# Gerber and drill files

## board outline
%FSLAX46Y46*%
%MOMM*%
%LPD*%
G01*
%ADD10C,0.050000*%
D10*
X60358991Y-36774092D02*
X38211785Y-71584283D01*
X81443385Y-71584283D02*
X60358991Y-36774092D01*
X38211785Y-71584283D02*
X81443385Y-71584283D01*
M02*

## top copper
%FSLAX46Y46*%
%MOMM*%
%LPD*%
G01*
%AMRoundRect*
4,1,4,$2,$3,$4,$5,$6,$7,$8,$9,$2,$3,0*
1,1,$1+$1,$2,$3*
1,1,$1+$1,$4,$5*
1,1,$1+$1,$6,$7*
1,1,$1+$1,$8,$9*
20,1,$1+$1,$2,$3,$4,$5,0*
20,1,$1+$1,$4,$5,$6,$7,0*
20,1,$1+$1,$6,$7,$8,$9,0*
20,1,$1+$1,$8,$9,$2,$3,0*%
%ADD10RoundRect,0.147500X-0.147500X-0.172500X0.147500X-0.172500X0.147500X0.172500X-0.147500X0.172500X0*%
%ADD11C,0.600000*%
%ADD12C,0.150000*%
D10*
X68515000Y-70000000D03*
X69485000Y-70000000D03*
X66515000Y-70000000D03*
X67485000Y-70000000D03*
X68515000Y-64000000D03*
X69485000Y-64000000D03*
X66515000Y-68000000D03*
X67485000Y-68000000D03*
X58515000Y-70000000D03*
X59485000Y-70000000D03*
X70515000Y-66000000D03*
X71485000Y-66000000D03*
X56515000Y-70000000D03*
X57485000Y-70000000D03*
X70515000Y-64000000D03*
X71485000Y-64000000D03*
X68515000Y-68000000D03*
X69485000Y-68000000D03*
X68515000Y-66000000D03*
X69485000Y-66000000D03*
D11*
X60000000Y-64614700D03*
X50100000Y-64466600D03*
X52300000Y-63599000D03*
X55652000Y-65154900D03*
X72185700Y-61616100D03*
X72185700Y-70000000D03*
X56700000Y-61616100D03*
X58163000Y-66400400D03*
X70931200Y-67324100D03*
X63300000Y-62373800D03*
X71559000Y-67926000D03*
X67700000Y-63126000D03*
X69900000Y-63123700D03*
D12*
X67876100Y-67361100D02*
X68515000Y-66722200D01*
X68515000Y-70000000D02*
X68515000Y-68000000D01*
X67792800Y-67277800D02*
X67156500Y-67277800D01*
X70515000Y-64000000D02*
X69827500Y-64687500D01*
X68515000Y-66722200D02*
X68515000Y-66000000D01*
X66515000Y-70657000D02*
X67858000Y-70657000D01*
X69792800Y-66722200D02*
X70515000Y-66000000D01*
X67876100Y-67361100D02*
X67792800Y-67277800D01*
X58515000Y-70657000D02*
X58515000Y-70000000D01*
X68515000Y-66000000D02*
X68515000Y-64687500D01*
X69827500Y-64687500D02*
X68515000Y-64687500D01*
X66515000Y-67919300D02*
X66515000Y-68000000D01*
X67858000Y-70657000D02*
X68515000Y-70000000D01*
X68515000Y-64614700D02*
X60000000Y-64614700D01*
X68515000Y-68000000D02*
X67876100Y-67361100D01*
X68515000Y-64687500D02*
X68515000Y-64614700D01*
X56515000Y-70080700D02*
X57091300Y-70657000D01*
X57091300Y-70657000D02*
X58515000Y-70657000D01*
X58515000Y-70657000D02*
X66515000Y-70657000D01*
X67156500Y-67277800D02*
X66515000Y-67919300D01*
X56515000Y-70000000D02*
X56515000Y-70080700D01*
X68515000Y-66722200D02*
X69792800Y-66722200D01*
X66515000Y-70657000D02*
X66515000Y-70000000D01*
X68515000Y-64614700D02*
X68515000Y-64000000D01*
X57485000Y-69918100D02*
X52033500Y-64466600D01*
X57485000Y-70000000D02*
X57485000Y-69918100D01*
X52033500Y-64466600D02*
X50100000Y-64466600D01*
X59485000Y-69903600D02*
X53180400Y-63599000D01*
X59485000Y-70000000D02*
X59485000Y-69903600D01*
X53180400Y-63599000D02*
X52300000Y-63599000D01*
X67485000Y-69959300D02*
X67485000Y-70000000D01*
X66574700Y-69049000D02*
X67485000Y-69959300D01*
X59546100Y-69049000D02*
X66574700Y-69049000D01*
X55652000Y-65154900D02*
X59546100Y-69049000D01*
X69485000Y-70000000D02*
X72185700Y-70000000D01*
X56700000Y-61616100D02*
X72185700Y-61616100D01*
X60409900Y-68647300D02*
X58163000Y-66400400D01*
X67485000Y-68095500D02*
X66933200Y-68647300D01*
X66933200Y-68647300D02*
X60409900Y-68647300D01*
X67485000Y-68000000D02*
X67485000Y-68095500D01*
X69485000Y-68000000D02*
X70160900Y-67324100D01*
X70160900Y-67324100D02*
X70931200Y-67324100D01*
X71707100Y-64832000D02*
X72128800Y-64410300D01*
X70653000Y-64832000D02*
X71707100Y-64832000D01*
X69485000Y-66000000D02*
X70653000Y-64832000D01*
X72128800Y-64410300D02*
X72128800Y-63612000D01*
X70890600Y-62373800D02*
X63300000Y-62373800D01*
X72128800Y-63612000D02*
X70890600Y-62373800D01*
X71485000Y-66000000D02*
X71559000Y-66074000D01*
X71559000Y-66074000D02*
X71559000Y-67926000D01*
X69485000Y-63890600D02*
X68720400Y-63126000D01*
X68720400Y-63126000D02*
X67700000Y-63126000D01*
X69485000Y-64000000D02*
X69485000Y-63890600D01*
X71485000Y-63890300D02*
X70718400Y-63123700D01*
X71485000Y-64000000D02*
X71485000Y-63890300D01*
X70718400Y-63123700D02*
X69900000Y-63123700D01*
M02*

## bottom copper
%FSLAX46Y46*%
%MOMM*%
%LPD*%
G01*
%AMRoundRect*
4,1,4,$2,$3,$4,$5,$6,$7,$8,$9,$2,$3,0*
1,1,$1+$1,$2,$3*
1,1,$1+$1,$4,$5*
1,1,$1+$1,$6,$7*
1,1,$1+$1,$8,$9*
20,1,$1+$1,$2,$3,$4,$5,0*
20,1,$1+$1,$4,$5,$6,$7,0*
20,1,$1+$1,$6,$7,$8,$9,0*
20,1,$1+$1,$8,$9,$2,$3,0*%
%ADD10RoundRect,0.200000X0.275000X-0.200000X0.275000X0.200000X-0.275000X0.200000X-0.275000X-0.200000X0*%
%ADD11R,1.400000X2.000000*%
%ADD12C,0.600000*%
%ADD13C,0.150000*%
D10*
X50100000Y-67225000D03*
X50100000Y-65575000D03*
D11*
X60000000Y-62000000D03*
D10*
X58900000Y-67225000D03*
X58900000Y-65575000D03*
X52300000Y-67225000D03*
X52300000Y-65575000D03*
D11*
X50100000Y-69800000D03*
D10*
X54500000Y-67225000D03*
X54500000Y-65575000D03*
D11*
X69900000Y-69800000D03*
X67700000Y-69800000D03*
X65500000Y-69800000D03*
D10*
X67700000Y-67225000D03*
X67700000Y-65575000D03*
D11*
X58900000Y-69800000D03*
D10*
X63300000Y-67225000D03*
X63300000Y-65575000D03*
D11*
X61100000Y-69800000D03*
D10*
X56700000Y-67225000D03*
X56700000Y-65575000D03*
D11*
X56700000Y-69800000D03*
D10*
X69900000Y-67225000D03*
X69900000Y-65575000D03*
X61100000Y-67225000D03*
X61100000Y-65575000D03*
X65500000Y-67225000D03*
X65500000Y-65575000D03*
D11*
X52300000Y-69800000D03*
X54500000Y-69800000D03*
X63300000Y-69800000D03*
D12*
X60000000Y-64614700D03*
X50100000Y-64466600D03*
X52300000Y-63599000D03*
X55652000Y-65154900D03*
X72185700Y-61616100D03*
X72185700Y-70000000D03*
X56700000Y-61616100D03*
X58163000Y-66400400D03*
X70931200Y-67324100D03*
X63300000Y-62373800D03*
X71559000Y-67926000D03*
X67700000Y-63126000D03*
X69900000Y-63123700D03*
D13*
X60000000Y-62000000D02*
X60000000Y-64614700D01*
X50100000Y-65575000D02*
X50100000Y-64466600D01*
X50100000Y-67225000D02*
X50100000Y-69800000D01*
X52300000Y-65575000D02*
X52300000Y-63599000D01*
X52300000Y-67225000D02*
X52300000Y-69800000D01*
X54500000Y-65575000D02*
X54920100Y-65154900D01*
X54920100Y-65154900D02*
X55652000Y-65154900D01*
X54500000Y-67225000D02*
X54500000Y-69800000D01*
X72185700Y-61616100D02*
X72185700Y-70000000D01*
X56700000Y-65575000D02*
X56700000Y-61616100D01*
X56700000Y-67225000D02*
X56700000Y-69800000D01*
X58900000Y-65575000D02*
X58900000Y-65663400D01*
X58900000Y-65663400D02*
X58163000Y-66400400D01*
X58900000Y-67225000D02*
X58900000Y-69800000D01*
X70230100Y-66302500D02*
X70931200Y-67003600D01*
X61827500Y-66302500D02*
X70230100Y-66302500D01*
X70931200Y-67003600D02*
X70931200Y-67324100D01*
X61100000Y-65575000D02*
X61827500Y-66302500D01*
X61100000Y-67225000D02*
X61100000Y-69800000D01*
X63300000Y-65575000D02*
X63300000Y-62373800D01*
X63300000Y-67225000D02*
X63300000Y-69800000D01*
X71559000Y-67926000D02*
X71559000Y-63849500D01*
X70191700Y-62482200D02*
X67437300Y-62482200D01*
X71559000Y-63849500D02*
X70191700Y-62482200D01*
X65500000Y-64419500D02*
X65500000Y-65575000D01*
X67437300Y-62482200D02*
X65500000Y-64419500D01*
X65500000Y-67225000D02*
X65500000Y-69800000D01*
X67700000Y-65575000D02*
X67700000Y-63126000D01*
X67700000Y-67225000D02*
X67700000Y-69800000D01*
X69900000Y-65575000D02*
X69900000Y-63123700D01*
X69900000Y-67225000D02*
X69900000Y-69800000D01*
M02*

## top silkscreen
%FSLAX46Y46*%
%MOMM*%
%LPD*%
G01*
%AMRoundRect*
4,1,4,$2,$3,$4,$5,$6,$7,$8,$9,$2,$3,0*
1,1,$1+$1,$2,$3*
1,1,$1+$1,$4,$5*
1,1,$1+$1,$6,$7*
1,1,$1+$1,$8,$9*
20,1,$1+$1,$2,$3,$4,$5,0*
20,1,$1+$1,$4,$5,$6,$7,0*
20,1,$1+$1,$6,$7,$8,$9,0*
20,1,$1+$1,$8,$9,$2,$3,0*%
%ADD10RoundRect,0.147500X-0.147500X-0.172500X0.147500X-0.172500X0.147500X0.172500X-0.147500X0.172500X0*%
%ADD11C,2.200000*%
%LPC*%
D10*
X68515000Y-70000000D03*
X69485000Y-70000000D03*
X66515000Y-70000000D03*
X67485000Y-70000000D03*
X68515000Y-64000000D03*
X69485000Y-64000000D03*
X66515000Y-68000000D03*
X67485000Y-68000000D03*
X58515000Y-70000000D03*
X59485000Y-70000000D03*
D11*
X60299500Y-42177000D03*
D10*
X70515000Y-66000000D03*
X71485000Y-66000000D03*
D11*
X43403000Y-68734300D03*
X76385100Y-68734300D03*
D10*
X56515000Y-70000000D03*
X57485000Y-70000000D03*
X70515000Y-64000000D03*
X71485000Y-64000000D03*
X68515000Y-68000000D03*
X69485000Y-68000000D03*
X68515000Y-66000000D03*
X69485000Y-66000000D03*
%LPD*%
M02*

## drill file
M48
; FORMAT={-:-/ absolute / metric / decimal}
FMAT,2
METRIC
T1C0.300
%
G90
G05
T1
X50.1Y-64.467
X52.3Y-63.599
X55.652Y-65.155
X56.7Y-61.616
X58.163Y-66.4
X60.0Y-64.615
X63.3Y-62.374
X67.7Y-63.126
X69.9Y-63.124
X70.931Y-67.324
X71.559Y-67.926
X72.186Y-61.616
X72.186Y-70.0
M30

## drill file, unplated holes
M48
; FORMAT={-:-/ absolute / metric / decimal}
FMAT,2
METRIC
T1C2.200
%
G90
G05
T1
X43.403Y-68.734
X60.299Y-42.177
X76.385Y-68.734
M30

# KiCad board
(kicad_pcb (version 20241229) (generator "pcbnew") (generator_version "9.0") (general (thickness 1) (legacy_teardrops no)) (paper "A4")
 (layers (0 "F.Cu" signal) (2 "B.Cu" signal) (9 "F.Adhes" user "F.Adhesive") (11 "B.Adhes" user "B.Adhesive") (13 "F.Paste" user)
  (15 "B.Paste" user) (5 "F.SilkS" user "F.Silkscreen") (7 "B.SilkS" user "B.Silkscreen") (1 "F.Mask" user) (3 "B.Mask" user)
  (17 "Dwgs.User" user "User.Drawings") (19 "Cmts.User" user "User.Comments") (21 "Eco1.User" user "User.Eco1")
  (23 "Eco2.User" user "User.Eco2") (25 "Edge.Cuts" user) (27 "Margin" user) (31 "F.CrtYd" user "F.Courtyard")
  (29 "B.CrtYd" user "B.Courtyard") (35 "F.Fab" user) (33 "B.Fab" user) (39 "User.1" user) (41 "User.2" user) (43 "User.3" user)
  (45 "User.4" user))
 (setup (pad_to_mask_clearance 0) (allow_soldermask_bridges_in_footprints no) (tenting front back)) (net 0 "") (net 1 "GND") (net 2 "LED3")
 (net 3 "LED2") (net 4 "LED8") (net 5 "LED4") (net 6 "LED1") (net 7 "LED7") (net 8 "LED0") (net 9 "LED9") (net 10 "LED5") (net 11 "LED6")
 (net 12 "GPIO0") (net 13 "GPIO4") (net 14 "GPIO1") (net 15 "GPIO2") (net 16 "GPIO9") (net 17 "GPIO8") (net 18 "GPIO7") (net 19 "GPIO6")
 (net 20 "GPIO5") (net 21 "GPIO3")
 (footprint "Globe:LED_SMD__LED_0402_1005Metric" (layer "F.Cu") (at 69 70)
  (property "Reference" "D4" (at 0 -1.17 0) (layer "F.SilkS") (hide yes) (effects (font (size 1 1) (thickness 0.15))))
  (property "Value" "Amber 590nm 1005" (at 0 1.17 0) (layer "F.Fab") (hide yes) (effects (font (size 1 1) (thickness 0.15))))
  (pad "1" smd roundrect (at -0.485 0) (size 0.59 0.64) (layers "F.Cu" "F.Mask" "F.Paste") (roundrect_rratio 0.25) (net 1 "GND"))
  (pad "2" smd roundrect (at 0.485 0) (size 0.59 0.64) (layers "F.Cu" "F.Mask" "F.Paste") (roundrect_rratio 0.25) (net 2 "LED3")))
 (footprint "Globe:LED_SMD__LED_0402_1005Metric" (layer "F.Cu") (at 67 70)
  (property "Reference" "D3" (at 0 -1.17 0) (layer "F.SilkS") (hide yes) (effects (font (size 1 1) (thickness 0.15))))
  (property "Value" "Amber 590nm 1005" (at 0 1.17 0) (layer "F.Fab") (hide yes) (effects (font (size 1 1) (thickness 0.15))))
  (pad "1" smd roundrect (at -0.485 0) (size 0.59 0.64) (layers "F.Cu" "F.Mask" "F.Paste") (roundrect_rratio 0.25) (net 1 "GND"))
  (pad "2" smd roundrect (at 0.485 0) (size 0.59 0.64) (layers "F.Cu" "F.Mask" "F.Paste") (roundrect_rratio 0.25) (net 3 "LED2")))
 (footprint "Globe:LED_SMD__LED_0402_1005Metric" (layer "F.Cu") (at 69 64)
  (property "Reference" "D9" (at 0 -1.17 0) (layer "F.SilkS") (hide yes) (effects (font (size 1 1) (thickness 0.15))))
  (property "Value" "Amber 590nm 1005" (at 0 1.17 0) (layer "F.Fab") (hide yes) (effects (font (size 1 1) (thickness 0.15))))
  (pad "1" smd roundrect (at -0.485 0) (size 0.59 0.64) (layers "F.Cu" "F.Mask" "F.Paste") (roundrect_rratio 0.25) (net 1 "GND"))
  (pad "2" smd roundrect (at 0.485 0) (size 0.59 0.64) (layers "F.Cu" "F.Mask" "F.Paste") (roundrect_rratio 0.25) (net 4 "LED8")))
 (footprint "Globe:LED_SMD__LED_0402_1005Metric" (layer "F.Cu") (at 67 68)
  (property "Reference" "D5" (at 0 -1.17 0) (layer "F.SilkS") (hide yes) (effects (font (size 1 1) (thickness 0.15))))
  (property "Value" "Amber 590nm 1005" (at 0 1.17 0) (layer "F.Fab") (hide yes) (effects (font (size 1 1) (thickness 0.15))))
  (pad "1" smd roundrect (at -0.485 0) (size 0.59 0.64) (layers "F.Cu" "F.Mask" "F.Paste") (roundrect_rratio 0.25) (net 1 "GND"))
  (pad "2" smd roundrect (at 0.485 0) (size 0.59 0.64) (layers "F.Cu" "F.Mask" "F.Paste") (roundrect_rratio 0.25) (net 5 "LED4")))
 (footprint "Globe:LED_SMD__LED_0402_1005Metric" (layer "F.Cu") (at 59 70)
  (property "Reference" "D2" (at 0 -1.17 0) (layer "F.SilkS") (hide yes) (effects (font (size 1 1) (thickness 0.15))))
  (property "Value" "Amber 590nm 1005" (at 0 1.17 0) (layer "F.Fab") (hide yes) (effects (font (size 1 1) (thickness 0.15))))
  (pad "1" smd roundrect (at -0.485 0) (size 0.59 0.64) (layers "F.Cu" "F.Mask" "F.Paste") (roundrect_rratio 0.25) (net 1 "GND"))
  (pad "2" smd roundrect (at 0.485 0) (size 0.59 0.64) (layers "F.Cu" "F.Mask" "F.Paste") (roundrect_rratio 0.25) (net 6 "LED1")))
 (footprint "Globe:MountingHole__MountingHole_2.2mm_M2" (layer "F.Cu") (at 60.2995 42.177)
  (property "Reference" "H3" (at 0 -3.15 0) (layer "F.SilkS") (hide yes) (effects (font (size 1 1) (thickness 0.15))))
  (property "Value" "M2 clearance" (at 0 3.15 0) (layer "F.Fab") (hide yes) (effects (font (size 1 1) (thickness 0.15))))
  (pad "" np_thru_hole circle (at 0 0) (size 2.2 2.2) (drill 2.2) (layers "*.Cu" "*.Mask")))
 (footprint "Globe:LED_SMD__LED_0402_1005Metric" (layer "F.Cu") (at 71 66)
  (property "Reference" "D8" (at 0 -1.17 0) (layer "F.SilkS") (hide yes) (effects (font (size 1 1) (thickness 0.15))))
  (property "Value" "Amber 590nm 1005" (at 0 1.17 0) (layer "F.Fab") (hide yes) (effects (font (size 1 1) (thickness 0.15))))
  (pad "1" smd roundrect (at -0.485 0) (size 0.59 0.64) (layers "F.Cu" "F.Mask" "F.Paste") (roundrect_rratio 0.25) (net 1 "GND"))
  (pad "2" smd roundrect (at 0.485 0) (size 0.59 0.64) (layers "F.Cu" "F.Mask" "F.Paste") (roundrect_rratio 0.25) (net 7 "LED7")))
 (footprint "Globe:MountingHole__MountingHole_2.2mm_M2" (layer "F.Cu") (at 43.403 68.7343)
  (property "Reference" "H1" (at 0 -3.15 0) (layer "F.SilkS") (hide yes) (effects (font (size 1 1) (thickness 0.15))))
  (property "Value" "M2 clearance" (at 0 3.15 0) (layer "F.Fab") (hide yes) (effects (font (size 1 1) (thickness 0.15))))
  (pad "" np_thru_hole circle (at 0 0) (size 2.2 2.2) (drill 2.2) (layers "*.Cu" "*.Mask")))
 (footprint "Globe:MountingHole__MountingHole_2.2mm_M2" (layer "F.Cu") (at 76.3851 68.7343)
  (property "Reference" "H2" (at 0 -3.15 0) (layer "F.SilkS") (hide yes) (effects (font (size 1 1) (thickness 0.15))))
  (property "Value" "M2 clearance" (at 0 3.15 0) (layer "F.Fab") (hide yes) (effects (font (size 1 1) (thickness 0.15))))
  (pad "" np_thru_hole circle (at 0 0) (size 2.2 2.2) (drill 2.2) (layers "*.Cu" "*.Mask")))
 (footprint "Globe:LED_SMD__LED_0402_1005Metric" (layer "F.Cu") (at 57 70)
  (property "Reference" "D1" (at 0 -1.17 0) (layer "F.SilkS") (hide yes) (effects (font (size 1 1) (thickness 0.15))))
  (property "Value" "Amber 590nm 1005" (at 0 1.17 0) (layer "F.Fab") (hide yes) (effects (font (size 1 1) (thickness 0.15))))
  (pad "1" smd roundrect (at -0.485 0) (size 0.59 0.64) (layers "F.Cu" "F.Mask" "F.Paste") (roundrect_rratio 0.25) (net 1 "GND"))
  (pad "2" smd roundrect (at 0.485 0) (size 0.59 0.64) (layers "F.Cu" "F.Mask" "F.Paste") (roundrect_rratio 0.25) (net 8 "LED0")))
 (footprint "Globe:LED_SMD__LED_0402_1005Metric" (layer "F.Cu") (at 71 64)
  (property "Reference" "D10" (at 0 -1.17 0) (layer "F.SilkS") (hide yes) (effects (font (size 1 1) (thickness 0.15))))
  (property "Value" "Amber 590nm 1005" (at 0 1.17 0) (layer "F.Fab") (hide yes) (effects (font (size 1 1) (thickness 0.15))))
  (pad "1" smd roundrect (at -0.485 0) (size 0.59 0.64) (layers "F.Cu" "F.Mask" "F.Paste") (roundrect_rratio 0.25) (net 1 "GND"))
  (pad "2" smd roundrect (at 0.485 0) (size 0.59 0.64) (layers "F.Cu" "F.Mask" "F.Paste") (roundrect_rratio 0.25) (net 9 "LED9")))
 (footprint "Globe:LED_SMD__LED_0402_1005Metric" (layer "F.Cu") (at 69 68)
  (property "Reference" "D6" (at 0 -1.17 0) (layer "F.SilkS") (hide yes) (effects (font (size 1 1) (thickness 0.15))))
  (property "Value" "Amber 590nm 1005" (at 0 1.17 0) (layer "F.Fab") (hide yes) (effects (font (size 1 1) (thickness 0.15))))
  (pad "1" smd roundrect (at -0.485 0) (size 0.59 0.64) (layers "F.Cu" "F.Mask" "F.Paste") (roundrect_rratio 0.25) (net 1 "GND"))
  (pad "2" smd roundrect (at 0.485 0) (size 0.59 0.64) (layers "F.Cu" "F.Mask" "F.Paste") (roundrect_rratio 0.25) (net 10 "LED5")))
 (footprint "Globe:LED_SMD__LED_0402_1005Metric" (layer "F.Cu") (at 69 66)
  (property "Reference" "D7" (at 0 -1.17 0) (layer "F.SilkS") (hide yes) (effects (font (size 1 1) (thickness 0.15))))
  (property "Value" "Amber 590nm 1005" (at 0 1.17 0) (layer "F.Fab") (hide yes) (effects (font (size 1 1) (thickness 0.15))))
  (pad "1" smd roundrect (at -0.485 0) (size 0.59 0.64) (layers "F.Cu" "F.Mask" "F.Paste") (roundrect_rratio 0.25) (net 1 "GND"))
  (pad "2" smd roundrect (at 0.485 0) (size 0.59 0.64) (layers "F.Cu" "F.Mask" "F.Paste") (roundrect_rratio 0.25) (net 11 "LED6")))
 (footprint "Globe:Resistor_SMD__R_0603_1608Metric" (layer "B.Cu") (at 50.1 66.4 90)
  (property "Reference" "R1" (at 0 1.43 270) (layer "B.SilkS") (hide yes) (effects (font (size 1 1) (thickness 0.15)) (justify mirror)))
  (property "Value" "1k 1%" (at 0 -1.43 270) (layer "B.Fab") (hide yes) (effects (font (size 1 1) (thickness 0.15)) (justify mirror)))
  (pad "1" smd roundrect (at -0.825 0 90) (size 0.8 0.95) (layers "B.Cu" "B.Mask" "B.Paste") (roundrect_rratio 0.25) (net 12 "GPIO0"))
  (pad "2" smd roundrect (at 0.825 0 90) (size 0.8 0.95) (layers "B.Cu" "B.Mask" "B.Paste") (roundrect_rratio 0.25) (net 8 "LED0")))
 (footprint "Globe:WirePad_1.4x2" (layer "B.Cu") (at 60 62 180)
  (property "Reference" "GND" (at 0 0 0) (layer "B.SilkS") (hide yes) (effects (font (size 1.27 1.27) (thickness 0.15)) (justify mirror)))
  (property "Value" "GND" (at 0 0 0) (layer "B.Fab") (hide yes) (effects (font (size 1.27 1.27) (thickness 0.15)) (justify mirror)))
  (pad "1" smd rect (at 0 0 180) (size 1.4 2) (layers "B.Cu" "B.Mask") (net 1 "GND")))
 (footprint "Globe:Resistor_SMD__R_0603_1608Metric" (layer "B.Cu") (at 58.9 66.4 90)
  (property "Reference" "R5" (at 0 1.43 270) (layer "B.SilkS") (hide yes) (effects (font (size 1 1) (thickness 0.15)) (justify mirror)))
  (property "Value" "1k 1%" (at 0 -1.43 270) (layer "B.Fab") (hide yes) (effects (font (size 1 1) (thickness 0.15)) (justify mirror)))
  (pad "1" smd roundrect (at -0.825 0 90) (size 0.8 0.95) (layers "B.Cu" "B.Mask" "B.Paste") (roundrect_rratio 0.25) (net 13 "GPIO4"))
  (pad "2" smd roundrect (at 0.825 0 90) (size 0.8 0.95) (layers "B.Cu" "B.Mask" "B.Paste") (roundrect_rratio 0.25) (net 5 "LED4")))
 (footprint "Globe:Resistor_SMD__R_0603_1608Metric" (layer "B.Cu") (at 52.3 66.4 90)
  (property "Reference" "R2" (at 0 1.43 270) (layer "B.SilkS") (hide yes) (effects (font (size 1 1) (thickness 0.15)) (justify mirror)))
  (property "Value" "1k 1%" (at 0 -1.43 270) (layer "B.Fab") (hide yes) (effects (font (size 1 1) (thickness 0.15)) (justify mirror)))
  (pad "1" smd roundrect (at -0.825 0 90) (size 0.8 0.95) (layers "B.Cu" "B.Mask" "B.Paste") (roundrect_rratio 0.25) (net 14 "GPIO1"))
  (pad "2" smd roundrect (at 0.825 0 90) (size 0.8 0.95) (layers "B.Cu" "B.Mask" "B.Paste") (roundrect_rratio 0.25) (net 6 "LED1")))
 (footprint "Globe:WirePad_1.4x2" (layer "B.Cu") (at 50.1 69.8 180)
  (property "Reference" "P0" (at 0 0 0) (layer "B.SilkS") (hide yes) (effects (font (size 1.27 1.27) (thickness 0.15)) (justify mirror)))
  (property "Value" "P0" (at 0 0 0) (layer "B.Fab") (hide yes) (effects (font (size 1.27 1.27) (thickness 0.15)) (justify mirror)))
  (pad "1" smd rect (at 0 0 180) (size 1.4 2) (layers "B.Cu" "B.Mask") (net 12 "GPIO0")))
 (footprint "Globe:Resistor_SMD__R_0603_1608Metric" (layer "B.Cu") (at 54.5 66.4 90)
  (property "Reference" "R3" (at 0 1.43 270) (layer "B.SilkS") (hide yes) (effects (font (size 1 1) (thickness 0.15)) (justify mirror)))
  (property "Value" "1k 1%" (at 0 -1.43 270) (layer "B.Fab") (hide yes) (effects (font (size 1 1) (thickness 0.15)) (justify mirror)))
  (pad "1" smd roundrect (at -0.825 0 90) (size 0.8 0.95) (layers "B.Cu" "B.Mask" "B.Paste") (roundrect_rratio 0.25) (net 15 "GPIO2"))
  (pad "2" smd roundrect (at 0.825 0 90) (size 0.8 0.95) (layers "B.Cu" "B.Mask" "B.Paste") (roundrect_rratio 0.25) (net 3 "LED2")))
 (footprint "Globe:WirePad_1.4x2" (layer "B.Cu") (at 69.9 69.8 180)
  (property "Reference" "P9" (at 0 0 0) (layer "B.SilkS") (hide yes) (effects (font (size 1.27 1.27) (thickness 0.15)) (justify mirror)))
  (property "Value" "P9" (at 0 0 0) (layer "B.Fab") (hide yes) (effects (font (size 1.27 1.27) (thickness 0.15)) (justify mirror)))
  (pad "1" smd rect (at 0 0 180) (size 1.4 2) (layers "B.Cu" "B.Mask") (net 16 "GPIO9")))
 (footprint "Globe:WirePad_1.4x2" (layer "B.Cu") (at 67.7 69.8 180)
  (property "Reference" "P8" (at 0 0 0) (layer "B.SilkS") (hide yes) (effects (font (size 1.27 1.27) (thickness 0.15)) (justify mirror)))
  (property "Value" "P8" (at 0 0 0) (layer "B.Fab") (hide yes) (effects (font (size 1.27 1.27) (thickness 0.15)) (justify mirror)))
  (pad "1" smd rect (at 0 0 180) (size 1.4 2) (layers "B.Cu" "B.Mask") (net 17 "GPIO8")))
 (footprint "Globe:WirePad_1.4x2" (layer "B.Cu") (at 65.5 69.8 180)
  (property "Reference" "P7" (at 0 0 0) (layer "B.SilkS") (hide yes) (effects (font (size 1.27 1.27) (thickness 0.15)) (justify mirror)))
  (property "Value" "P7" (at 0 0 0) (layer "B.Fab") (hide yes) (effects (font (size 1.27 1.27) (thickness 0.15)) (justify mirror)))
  (pad "1" smd rect (at 0 0 180) (size 1.4 2) (layers "B.Cu" "B.Mask") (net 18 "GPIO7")))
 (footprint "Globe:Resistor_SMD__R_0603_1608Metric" (layer "B.Cu") (at 67.7 66.4 90)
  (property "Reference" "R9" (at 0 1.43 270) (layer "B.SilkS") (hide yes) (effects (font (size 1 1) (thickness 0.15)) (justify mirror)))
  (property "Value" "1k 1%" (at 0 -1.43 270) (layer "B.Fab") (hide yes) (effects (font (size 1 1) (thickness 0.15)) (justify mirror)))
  (pad "1" smd roundrect (at -0.825 0 90) (size 0.8 0.95) (layers "B.Cu" "B.Mask" "B.Paste") (roundrect_rratio 0.25) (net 17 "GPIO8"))
  (pad "2" smd roundrect (at 0.825 0 90) (size 0.8 0.95) (layers "B.Cu" "B.Mask" "B.Paste") (roundrect_rratio 0.25) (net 4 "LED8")))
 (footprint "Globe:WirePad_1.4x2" (layer "B.Cu") (at 58.9 69.8 180)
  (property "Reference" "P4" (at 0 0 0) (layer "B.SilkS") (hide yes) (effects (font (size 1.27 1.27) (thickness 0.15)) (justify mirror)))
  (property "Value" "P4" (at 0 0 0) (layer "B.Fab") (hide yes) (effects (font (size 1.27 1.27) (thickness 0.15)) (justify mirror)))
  (pad "1" smd rect (at 0 0 180) (size 1.4 2) (layers "B.Cu" "B.Mask") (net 13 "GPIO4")))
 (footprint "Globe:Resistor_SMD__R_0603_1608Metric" (layer "B.Cu") (at 63.3 66.4 90)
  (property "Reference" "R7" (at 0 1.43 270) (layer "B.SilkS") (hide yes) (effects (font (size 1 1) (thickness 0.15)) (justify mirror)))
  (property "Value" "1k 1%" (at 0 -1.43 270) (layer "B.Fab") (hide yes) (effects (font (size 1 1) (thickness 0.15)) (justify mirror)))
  (pad "1" smd roundrect (at -0.825 0 90) (size 0.8 0.95) (layers "B.Cu" "B.Mask" "B.Paste") (roundrect_rratio 0.25) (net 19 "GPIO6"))
  (pad "2" smd roundrect (at 0.825 0 90) (size 0.8 0.95) (layers "B.Cu" "B.Mask" "B.Paste") (roundrect_rratio 0.25) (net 11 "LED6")))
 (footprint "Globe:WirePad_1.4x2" (layer "B.Cu") (at 61.1 69.8 180)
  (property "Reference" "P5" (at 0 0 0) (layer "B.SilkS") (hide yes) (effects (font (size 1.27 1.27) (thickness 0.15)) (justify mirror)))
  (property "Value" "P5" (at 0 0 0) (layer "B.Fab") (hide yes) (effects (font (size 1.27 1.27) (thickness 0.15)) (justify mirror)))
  (pad "1" smd rect (at 0 0 180) (size 1.4 2) (layers "B.Cu" "B.Mask") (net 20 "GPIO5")))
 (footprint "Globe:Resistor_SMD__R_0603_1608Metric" (layer "B.Cu") (at 56.7 66.4 90)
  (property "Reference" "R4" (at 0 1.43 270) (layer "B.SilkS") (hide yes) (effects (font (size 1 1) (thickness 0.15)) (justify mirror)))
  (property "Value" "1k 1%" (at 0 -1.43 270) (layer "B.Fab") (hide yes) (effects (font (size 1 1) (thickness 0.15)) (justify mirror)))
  (pad "1" smd roundrect (at -0.825 0 90) (size 0.8 0.95) (layers "B.Cu" "B.Mask" "B.Paste") (roundrect_rratio 0.25) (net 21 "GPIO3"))
  (pad "2" smd roundrect (at 0.825 0 90) (size 0.8 0.95) (layers "B.Cu" "B.Mask" "B.Paste") (roundrect_rratio 0.25) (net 2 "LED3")))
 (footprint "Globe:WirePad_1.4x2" (layer "B.Cu") (at 56.7 69.8 180)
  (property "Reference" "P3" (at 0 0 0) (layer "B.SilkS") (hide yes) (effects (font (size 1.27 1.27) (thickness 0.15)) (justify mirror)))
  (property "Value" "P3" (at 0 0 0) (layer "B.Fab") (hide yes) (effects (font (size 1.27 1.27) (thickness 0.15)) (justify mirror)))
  (pad "1" smd rect (at 0 0 180) (size 1.4 2) (layers "B.Cu" "B.Mask") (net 21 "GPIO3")))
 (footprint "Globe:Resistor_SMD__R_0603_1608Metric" (layer "B.Cu") (at 69.9 66.4 90)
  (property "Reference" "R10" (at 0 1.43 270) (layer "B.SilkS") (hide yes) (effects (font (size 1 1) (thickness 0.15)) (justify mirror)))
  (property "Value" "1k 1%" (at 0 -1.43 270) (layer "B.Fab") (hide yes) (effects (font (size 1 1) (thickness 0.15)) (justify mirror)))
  (pad "1" smd roundrect (at -0.825 0 90) (size 0.8 0.95) (layers "B.Cu" "B.Mask" "B.Paste") (roundrect_rratio 0.25) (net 16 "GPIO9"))
  (pad "2" smd roundrect (at 0.825 0 90) (size 0.8 0.95) (layers "B.Cu" "B.Mask" "B.Paste") (roundrect_rratio 0.25) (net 9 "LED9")))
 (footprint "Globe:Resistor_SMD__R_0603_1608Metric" (layer "B.Cu") (at 61.1 66.4 90)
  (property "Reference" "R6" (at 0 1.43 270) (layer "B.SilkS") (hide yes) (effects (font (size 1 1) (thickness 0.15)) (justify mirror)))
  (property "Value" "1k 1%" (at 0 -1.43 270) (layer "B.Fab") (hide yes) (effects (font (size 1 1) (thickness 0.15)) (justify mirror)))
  (pad "1" smd roundrect (at -0.825 0 90) (size 0.8 0.95) (layers "B.Cu" "B.Mask" "B.Paste") (roundrect_rratio 0.25) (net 20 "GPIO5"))
  (pad "2" smd roundrect (at 0.825 0 90) (size 0.8 0.95) (layers "B.Cu" "B.Mask" "B.Paste") (roundrect_rratio 0.25) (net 10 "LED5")))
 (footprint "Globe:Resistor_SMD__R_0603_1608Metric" (layer "B.Cu") (at 65.5 66.4 90)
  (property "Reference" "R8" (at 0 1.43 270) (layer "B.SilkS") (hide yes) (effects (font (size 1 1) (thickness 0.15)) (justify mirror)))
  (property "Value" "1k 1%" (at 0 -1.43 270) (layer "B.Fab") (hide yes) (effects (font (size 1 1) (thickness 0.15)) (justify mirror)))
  (pad "1" smd roundrect (at -0.825 0 90) (size 0.8 0.95) (layers "B.Cu" "B.Mask" "B.Paste") (roundrect_rratio 0.25) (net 18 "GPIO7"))
  (pad "2" smd roundrect (at 0.825 0 90) (size 0.8 0.95) (layers "B.Cu" "B.Mask" "B.Paste") (roundrect_rratio 0.25) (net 7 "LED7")))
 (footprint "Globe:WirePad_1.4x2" (layer "B.Cu") (at 52.3 69.8 180)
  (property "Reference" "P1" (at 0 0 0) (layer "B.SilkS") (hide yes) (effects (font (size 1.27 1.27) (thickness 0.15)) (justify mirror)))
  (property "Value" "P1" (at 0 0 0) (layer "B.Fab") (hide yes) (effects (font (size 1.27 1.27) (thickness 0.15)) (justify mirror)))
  (pad "1" smd rect (at 0 0 180) (size 1.4 2) (layers "B.Cu" "B.Mask") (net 14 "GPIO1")))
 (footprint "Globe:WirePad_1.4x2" (layer "B.Cu") (at 54.5 69.8 180)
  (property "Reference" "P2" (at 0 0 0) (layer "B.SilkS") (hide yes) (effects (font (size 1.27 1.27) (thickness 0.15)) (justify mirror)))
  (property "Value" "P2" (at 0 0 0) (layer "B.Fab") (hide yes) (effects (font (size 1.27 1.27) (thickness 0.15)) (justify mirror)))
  (pad "1" smd rect (at 0 0 180) (size 1.4 2) (layers "B.Cu" "B.Mask") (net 15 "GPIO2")))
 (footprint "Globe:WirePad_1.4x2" (layer "B.Cu") (at 63.3 69.8 180)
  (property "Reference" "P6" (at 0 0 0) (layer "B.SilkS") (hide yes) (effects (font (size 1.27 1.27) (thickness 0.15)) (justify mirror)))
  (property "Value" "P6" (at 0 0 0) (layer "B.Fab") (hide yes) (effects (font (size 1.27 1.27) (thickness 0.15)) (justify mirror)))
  (pad "1" smd rect (at 0 0 180) (size 1.4 2) (layers "B.Cu" "B.Mask") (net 19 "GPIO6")))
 (gr_line (start 60.358991 36.774092) (end 38.211785 71.584283) (stroke (width 0.05) (type default)) (layer "Edge.Cuts"))
 (gr_line (start 81.443385 71.584283) (end 60.358991 36.774092) (stroke (width 0.05) (type default)) (layer "Edge.Cuts"))
 (gr_line (start 38.211785 71.584283) (end 81.443385 71.584283) (stroke (width 0.05) (type default)) (layer "Edge.Cuts"))
 (segment (start 67.8761 67.3611) (end 68.515 66.7222) (width 0.15) (layer "F.Cu") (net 1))
 (segment (start 68.515 70) (end 68.515 68) (width 0.15) (layer "F.Cu") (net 1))
 (segment (start 67.7928 67.2778) (end 67.1565 67.2778) (width 0.15) (layer "F.Cu") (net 1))
 (segment (start 70.515 64) (end 69.8275 64.6875) (width 0.15) (layer "F.Cu") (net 1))
 (segment (start 68.515 66.7222) (end 68.515 66) (width 0.15) (layer "F.Cu") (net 1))
 (segment (start 66.515 70.657) (end 67.858 70.657) (width 0.15) (layer "F.Cu") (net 1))
 (segment (start 69.7928 66.7222) (end 70.515 66) (width 0.15) (layer "F.Cu") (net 1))
 (segment (start 67.8761 67.3611) (end 67.7928 67.2778) (width 0.15) (layer "F.Cu") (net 1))
 (segment (start 58.515 70.657) (end 58.515 70) (width 0.15) (layer "F.Cu") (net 1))
 (segment (start 68.515 66) (end 68.515 64.6875) (width 0.15) (layer "F.Cu") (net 1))
 (segment (start 69.8275 64.6875) (end 68.515 64.6875) (width 0.15) (layer "F.Cu") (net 1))
 (segment (start 66.515 67.9193) (end 66.515 68) (width 0.15) (layer "F.Cu") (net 1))
 (segment (start 67.858 70.657) (end 68.515 70) (width 0.15) (layer "F.Cu") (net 1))
 (segment (start 68.515 64.6147) (end 60 64.6147) (width 0.15) (layer "F.Cu") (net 1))
 (segment (start 68.515 68) (end 67.8761 67.3611) (width 0.15) (layer "F.Cu") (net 1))
 (segment (start 68.515 64.6875) (end 68.515 64.6147) (width 0.15) (layer "F.Cu") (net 1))
 (segment (start 56.515 70.0807) (end 57.0913 70.657) (width 0.15) (layer "F.Cu") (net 1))
 (segment (start 57.0913 70.657) (end 58.515 70.657) (width 0.15) (layer "F.Cu") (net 1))
 (segment (start 58.515 70.657) (end 66.515 70.657) (width 0.15) (layer "F.Cu") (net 1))
 (segment (start 67.1565 67.2778) (end 66.515 67.9193) (width 0.15) (layer "F.Cu") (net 1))
 (segment (start 56.515 70) (end 56.515 70.0807) (width 0.15) (layer "F.Cu") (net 1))
 (segment (start 68.515 66.7222) (end 69.7928 66.7222) (width 0.15) (layer "F.Cu") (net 1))
 (segment (start 66.515 70.657) (end 66.515 70) (width 0.15) (layer "F.Cu") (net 1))
 (segment (start 68.515 64.6147) (end 68.515 64) (width 0.15) (layer "F.Cu") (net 1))
 (via (at 60 64.6147) (size 0.6) (drill 0.3) (layers "F.Cu" "B.Cu") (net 1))
 (segment (start 60 62) (end 60 64.6147) (width 0.15) (layer "B.Cu") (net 1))
 (segment (start 57.485 69.9181) (end 52.0335 64.4666) (width 0.15) (layer "F.Cu") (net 8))
 (segment (start 57.485 70) (end 57.485 69.9181) (width 0.15) (layer "F.Cu") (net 8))
 (segment (start 52.0335 64.4666) (end 50.1 64.4666) (width 0.15) (layer "F.Cu") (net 8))
 (via (at 50.1 64.4666) (size 0.6) (drill 0.3) (layers "F.Cu" "B.Cu") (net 8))
 (segment (start 50.1 65.575) (end 50.1 64.4666) (width 0.15) (layer "B.Cu") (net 8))
 (segment (start 50.1 67.225) (end 50.1 69.8) (width 0.15) (layer "B.Cu") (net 12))
 (segment (start 59.485 69.9036) (end 53.1804 63.599) (width 0.15) (layer "F.Cu") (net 6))
 (segment (start 59.485 70) (end 59.485 69.9036) (width 0.15) (layer "F.Cu") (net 6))
 (segment (start 53.1804 63.599) (end 52.3 63.599) (width 0.15) (layer "F.Cu") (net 6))
 (via (at 52.3 63.599) (size 0.6) (drill 0.3) (layers "F.Cu" "B.Cu") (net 6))
 (segment (start 52.3 65.575) (end 52.3 63.599) (width 0.15) (layer "B.Cu") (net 6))
 (segment (start 52.3 67.225) (end 52.3 69.8) (width 0.15) (layer "B.Cu") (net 14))
 (segment (start 67.485 69.9593) (end 67.485 70) (width 0.15) (layer "F.Cu") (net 3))
 (segment (start 66.5747 69.049) (end 67.485 69.9593) (width 0.15) (layer "F.Cu") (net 3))
 (segment (start 59.5461 69.049) (end 66.5747 69.049) (width 0.15) (layer "F.Cu") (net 3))
 (segment (start 55.652 65.1549) (end 59.5461 69.049) (width 0.15) (layer "F.Cu") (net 3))
 (via (at 55.652 65.1549) (size 0.6) (drill 0.3) (layers "F.Cu" "B.Cu") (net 3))
 (segment (start 54.5 65.575) (end 54.9201 65.1549) (width 0.15) (layer "B.Cu") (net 3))
 (segment (start 54.9201 65.1549) (end 55.652 65.1549) (width 0.15) (layer "B.Cu") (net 3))
 (segment (start 54.5 67.225) (end 54.5 69.8) (width 0.15) (layer "B.Cu") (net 15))
 (segment (start 69.485 70) (end 72.1857 70) (width 0.15) (layer "F.Cu") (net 2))
 (segment (start 56.7 61.6161) (end 72.1857 61.6161) (width 0.15) (layer "F.Cu") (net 2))
 (via (at 72.1857 61.6161) (size 0.6) (drill 0.3) (layers "F.Cu" "B.Cu") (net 2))
 (via (at 72.1857 70) (size 0.6) (drill 0.3) (layers "F.Cu" "B.Cu") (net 2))
 (via (at 56.7 61.6161) (size 0.6) (drill 0.3) (layers "F.Cu" "B.Cu") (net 2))
 (segment (start 72.1857 61.6161) (end 72.1857 70) (width 0.15) (layer "B.Cu") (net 2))
 (segment (start 56.7 65.575) (end 56.7 61.6161) (width 0.15) (layer "B.Cu") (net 2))
 (segment (start 56.7 67.225) (end 56.7 69.8) (width 0.15) (layer "B.Cu") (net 21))
 (segment (start 60.4099 68.6473) (end 58.163 66.4004) (width 0.15) (layer "F.Cu") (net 5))
 (segment (start 67.485 68.0955) (end 66.9332 68.6473) (width 0.15) (layer "F.Cu") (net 5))
 (segment (start 66.9332 68.6473) (end 60.4099 68.6473) (width 0.15) (layer "F.Cu") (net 5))
 (segment (start 67.485 68) (end 67.485 68.0955) (width 0.15) (layer "F.Cu") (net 5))
 (via (at 58.163 66.4004) (size 0.6) (drill 0.3) (layers "F.Cu" "B.Cu") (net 5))
 (segment (start 58.9 65.575) (end 58.9 65.6634) (width 0.15) (layer "B.Cu") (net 5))
 (segment (start 58.9 65.6634) (end 58.163 66.4004) (width 0.15) (layer "B.Cu") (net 5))
 (segment (start 58.9 67.225) (end 58.9 69.8) (width 0.15) (layer "B.Cu") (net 13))
 (segment (start 69.485 68) (end 70.1609 67.3241) (width 0.15) (layer "F.Cu") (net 10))
 (segment (start 70.1609 67.3241) (end 70.9312 67.3241) (width 0.15) (layer "F.Cu") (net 10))
 (via (at 70.9312 67.3241) (size 0.6) (drill 0.3) (layers "F.Cu" "B.Cu") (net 10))
 (segment (start 70.2301 66.3025) (end 70.9312 67.0036) (width 0.15) (layer "B.Cu") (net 10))
 (segment (start 61.8275 66.3025) (end 70.2301 66.3025) (width 0.15) (layer "B.Cu") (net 10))
 (segment (start 70.9312 67.0036) (end 70.9312 67.3241) (width 0.15) (layer "B.Cu") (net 10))
 (segment (start 61.1 65.575) (end 61.8275 66.3025) (width 0.15) (layer "B.Cu") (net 10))
 (segment (start 61.1 67.225) (end 61.1 69.8) (width 0.15) (layer "B.Cu") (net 20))
 (segment (start 71.7071 64.832) (end 72.1288 64.4103) (width 0.15) (layer "F.Cu") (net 11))
 (segment (start 70.653 64.832) (end 71.7071 64.832) (width 0.15) (layer "F.Cu") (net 11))
 (segment (start 69.485 66) (end 70.653 64.832) (width 0.15) (layer "F.Cu") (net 11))
 (segment (start 72.1288 64.4103) (end 72.1288 63.612) (width 0.15) (layer "F.Cu") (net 11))
 (segment (start 70.8906 62.3738) (end 63.3 62.3738) (width 0.15) (layer "F.Cu") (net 11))
 (segment (start 72.1288 63.612) (end 70.8906 62.3738) (width 0.15) (layer "F.Cu") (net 11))
 (via (at 63.3 62.3738) (size 0.6) (drill 0.3) (layers "F.Cu" "B.Cu") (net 11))
 (segment (start 63.3 65.575) (end 63.3 62.3738) (width 0.15) (layer "B.Cu") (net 11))
 (segment (start 63.3 67.225) (end 63.3 69.8) (width 0.15) (layer "B.Cu") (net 19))
 (segment (start 71.485 66) (end 71.559 66.074) (width 0.15) (layer "F.Cu") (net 7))
 (segment (start 71.559 66.074) (end 71.559 67.926) (width 0.15) (layer "F.Cu") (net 7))
 (via (at 71.559 67.926) (size 0.6) (drill 0.3) (layers "F.Cu" "B.Cu") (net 7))
 (segment (start 71.559 67.926) (end 71.559 63.8495) (width 0.15) (layer "B.Cu") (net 7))
 (segment (start 70.1917 62.4822) (end 67.4373 62.4822) (width 0.15) (layer "B.Cu") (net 7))
 (segment (start 71.559 63.8495) (end 70.1917 62.4822) (width 0.15) (layer "B.Cu") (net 7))
 (segment (start 65.5 64.4195) (end 65.5 65.575) (width 0.15) (layer "B.Cu") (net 7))
 (segment (start 67.4373 62.4822) (end 65.5 64.4195) (width 0.15) (layer "B.Cu") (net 7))
 (segment (start 65.5 67.225) (end 65.5 69.8) (width 0.15) (layer "B.Cu") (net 18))
 (segment (start 69.485 63.8906) (end 68.7204 63.126) (width 0.15) (layer "F.Cu") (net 4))
 (segment (start 68.7204 63.126) (end 67.7 63.126) (width 0.15) (layer "F.Cu") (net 4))
 (segment (start 69.485 64) (end 69.485 63.8906) (width 0.15) (layer "F.Cu") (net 4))
 (via (at 67.7 63.126) (size 0.6) (drill 0.3) (layers "F.Cu" "B.Cu") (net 4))
 (segment (start 67.7 65.575) (end 67.7 63.126) (width 0.15) (layer "B.Cu") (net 4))
 (segment (start 67.7 67.225) (end 67.7 69.8) (width 0.15) (layer "B.Cu") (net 17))
 (segment (start 71.485 63.8903) (end 70.7184 63.1237) (width 0.15) (layer "F.Cu") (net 9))
 (segment (start 71.485 64) (end 71.485 63.8903) (width 0.15) (layer "F.Cu") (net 9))
 (segment (start 70.7184 63.1237) (end 69.9 63.1237) (width 0.15) (layer "F.Cu") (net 9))
 (via (at 69.9 63.1237) (size 0.6) (drill 0.3) (layers "F.Cu" "B.Cu") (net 9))
 (segment (start 69.9 65.575) (end 69.9 63.1237) (width 0.15) (layer "B.Cu") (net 9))
 (segment (start 69.9 67.225) (end 69.9 69.8) (width 0.15) (layer "B.Cu") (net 16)))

